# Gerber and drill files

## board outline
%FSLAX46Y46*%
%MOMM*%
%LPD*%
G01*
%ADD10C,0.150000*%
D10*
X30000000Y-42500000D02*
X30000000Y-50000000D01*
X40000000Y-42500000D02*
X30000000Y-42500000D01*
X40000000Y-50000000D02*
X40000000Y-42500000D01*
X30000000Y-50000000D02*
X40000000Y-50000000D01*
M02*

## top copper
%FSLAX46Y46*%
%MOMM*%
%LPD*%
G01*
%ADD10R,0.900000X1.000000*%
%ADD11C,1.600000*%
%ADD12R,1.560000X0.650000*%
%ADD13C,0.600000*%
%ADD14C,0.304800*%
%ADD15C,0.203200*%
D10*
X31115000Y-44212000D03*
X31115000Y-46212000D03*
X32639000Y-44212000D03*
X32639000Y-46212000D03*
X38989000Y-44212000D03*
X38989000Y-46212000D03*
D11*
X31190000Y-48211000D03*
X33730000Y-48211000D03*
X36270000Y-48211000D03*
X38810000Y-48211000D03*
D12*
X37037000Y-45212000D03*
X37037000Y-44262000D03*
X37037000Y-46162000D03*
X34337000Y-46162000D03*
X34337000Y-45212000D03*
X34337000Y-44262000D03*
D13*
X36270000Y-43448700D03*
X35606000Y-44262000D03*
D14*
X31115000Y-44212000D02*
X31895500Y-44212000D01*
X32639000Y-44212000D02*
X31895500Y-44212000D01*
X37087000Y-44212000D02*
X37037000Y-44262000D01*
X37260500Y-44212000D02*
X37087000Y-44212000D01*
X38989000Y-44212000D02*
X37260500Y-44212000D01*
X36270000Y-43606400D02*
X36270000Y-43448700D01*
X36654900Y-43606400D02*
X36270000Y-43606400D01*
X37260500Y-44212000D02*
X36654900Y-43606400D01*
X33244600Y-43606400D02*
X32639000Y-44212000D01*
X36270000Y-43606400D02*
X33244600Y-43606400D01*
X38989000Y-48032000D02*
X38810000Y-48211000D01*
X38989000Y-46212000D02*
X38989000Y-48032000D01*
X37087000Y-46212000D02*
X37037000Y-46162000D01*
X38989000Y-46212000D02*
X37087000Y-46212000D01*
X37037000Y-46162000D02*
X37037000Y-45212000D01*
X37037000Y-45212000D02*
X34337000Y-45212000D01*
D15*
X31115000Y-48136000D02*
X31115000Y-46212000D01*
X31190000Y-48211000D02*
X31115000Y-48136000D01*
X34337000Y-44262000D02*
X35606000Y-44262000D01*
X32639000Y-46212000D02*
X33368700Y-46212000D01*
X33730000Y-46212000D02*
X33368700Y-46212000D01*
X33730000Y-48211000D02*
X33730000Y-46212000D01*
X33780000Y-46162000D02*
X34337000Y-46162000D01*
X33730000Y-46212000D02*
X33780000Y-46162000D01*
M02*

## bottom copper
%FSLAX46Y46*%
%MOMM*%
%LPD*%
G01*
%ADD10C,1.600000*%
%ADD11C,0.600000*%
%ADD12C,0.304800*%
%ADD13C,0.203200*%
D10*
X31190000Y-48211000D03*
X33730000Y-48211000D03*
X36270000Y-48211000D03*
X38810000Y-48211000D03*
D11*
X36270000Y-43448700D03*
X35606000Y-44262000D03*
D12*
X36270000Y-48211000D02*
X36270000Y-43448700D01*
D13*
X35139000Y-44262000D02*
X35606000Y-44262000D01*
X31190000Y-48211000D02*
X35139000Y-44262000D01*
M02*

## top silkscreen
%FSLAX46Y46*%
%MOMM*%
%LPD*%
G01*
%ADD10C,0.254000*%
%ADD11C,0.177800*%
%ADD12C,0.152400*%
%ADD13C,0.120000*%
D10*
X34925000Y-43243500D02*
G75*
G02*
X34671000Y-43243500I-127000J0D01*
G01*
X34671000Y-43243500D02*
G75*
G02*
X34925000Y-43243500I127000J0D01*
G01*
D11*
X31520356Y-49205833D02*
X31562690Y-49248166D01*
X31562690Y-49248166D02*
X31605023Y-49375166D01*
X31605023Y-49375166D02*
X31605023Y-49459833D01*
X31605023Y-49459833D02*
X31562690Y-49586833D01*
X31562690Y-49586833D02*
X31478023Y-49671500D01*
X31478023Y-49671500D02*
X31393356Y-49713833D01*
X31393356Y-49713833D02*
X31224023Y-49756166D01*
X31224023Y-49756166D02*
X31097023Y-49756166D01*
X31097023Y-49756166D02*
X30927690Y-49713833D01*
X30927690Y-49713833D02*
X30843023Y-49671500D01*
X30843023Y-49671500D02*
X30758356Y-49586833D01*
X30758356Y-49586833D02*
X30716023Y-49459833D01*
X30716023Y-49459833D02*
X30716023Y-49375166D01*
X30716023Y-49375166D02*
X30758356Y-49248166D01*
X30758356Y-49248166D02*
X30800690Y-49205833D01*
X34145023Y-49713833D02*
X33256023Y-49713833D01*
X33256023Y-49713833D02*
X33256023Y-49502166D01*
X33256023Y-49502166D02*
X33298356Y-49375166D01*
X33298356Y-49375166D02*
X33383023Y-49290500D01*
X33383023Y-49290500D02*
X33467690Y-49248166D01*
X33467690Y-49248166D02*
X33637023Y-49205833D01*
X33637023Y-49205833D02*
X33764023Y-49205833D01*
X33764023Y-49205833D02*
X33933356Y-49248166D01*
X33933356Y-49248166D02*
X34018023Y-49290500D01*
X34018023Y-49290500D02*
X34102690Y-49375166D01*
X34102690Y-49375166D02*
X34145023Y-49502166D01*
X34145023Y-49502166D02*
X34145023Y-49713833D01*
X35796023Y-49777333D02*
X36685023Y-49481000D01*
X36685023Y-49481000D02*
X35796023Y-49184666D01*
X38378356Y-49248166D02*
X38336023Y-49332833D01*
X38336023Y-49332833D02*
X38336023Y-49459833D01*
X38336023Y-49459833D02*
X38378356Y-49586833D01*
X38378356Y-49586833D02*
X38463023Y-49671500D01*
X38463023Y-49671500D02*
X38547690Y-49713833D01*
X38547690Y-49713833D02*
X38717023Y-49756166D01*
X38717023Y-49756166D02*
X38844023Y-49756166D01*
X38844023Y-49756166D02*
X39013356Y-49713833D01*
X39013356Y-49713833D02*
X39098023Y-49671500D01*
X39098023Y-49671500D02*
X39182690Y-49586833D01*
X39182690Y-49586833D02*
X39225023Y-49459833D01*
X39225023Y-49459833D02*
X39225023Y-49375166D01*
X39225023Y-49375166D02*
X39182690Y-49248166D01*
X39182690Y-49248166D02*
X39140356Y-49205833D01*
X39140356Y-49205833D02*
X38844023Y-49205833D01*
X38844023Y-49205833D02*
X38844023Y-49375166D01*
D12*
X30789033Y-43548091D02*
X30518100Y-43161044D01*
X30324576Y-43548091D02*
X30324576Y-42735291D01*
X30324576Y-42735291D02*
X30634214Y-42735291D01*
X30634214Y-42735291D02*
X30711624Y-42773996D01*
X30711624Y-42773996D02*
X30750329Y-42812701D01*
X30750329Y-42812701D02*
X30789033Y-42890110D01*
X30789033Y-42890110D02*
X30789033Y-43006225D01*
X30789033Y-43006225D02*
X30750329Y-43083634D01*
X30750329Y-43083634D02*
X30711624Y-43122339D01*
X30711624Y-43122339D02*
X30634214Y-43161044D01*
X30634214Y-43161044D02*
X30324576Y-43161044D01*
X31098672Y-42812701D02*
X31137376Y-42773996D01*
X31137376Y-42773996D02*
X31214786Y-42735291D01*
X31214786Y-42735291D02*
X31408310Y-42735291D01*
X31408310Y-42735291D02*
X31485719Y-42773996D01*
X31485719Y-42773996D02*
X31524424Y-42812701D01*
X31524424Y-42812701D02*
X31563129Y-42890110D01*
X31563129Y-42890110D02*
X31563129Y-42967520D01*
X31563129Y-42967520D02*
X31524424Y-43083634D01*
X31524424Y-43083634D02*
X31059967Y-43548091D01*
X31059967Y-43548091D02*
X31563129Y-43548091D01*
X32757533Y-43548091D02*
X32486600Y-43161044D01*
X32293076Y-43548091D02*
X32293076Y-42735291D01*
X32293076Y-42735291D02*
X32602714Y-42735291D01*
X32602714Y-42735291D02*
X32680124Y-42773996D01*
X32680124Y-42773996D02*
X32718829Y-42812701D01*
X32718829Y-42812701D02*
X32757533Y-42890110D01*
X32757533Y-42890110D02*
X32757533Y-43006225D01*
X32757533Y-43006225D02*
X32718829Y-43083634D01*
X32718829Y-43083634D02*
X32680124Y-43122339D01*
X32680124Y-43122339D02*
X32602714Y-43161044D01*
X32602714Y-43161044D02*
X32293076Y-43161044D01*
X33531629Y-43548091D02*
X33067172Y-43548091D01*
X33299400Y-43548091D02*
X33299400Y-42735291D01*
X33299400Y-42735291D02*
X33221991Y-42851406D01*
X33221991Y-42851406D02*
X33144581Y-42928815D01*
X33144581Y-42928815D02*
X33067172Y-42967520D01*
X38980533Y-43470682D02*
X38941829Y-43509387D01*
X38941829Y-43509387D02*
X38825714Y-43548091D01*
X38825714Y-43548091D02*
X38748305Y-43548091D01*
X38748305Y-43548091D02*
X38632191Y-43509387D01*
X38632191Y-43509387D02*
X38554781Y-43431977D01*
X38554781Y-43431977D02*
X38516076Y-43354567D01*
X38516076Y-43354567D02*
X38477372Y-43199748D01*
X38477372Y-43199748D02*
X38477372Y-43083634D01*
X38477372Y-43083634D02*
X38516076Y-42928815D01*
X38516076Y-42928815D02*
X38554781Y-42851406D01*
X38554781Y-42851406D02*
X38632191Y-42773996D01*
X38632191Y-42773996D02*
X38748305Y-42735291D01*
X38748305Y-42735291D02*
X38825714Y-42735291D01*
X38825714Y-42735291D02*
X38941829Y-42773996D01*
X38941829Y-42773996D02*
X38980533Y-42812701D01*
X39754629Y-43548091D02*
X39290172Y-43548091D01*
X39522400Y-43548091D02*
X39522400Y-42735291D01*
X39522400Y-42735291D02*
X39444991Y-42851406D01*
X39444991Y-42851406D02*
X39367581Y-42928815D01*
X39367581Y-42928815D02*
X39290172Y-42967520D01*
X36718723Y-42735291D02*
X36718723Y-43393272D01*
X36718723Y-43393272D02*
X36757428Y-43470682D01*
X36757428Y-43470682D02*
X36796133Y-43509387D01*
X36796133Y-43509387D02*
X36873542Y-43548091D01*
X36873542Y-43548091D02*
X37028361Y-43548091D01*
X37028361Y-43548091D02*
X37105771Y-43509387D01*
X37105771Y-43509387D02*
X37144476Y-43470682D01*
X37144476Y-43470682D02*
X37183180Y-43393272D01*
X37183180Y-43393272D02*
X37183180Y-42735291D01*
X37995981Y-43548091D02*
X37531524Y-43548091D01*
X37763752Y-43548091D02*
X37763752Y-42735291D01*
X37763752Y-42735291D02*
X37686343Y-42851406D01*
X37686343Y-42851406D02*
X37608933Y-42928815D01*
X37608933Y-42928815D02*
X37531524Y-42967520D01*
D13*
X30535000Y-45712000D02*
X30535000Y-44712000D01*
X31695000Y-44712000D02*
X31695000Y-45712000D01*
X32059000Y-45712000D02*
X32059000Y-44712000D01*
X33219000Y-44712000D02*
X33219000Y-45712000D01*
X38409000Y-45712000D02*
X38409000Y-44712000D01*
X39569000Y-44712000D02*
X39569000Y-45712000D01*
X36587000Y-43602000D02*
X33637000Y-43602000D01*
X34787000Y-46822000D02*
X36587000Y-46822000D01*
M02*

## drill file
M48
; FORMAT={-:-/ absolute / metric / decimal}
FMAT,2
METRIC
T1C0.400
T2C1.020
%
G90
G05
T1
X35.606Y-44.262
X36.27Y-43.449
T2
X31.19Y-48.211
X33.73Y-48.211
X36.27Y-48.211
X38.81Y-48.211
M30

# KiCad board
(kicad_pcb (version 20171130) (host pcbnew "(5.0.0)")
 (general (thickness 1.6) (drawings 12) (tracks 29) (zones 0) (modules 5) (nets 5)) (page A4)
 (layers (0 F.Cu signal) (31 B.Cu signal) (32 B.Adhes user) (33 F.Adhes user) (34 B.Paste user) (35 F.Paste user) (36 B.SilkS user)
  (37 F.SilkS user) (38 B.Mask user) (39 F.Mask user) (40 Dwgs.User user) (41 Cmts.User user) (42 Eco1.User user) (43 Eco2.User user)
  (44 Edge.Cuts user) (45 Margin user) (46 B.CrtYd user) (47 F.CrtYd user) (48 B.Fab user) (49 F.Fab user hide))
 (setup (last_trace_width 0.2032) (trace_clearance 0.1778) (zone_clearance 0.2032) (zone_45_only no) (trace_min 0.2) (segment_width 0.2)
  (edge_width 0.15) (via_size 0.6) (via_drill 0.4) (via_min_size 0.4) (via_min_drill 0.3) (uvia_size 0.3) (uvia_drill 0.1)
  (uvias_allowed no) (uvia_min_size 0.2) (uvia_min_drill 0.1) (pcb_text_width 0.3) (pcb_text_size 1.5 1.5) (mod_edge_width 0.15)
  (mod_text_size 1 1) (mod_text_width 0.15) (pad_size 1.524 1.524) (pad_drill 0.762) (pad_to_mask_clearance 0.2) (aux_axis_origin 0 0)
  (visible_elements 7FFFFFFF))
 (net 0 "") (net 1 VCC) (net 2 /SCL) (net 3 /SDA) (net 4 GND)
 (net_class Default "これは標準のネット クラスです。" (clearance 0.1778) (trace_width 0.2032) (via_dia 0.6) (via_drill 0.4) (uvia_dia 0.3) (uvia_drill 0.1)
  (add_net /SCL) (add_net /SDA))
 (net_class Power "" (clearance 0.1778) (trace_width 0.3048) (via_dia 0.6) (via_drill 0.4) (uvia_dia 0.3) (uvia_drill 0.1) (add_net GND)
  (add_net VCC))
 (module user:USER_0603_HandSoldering (layer F.Cu) (at 31.115 45.212 270)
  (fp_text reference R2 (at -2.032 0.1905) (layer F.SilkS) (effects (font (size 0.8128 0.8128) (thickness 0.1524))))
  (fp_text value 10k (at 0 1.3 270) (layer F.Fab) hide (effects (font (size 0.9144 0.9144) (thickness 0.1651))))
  (fp_line (start 0.5 0.58) (end -0.5 0.58) (layer F.SilkS) (width 0.12))
  (fp_line (start -0.5 -0.58) (end 0.5 -0.58) (layer F.SilkS) (width 0.12))
  (pad 1 smd rect (at -1 0 270) (size 1 0.9) (layers F.Cu F.Paste F.Mask) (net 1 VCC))
  (pad 2 smd rect (at 1 0 270) (size 1 0.9) (layers F.Cu F.Paste F.Mask) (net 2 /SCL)))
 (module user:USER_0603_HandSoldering (layer F.Cu) (at 32.639 45.212 270)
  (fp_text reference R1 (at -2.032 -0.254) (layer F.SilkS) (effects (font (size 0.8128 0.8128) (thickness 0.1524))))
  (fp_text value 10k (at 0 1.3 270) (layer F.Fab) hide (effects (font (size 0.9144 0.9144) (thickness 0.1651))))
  (fp_line (start 0.5 0.58) (end -0.5 0.58) (layer F.SilkS) (width 0.12))
  (fp_line (start -0.5 -0.58) (end 0.5 -0.58) (layer F.SilkS) (width 0.12))
  (pad 1 smd rect (at -1 0 270) (size 1 0.9) (layers F.Cu F.Paste F.Mask) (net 1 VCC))
  (pad 2 smd rect (at 1 0 270) (size 1 0.9) (layers F.Cu F.Paste F.Mask) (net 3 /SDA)))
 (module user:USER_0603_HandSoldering (layer F.Cu) (at 38.989 45.212 270)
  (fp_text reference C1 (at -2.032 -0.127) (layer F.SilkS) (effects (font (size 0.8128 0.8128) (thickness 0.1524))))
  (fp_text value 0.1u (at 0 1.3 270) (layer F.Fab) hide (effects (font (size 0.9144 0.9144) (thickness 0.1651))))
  (fp_line (start 0.5 0.58) (end -0.5 0.58) (layer F.SilkS) (width 0.12))
  (fp_line (start -0.5 -0.58) (end 0.5 -0.58) (layer F.SilkS) (width 0.12))
  (pad 1 smd rect (at -1 0 270) (size 1 0.9) (layers F.Cu F.Paste F.Mask) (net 1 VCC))
  (pad 2 smd rect (at 1 0 270) (size 1 0.9) (layers F.Cu F.Paste F.Mask) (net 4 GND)))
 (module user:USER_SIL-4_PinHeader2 (layer B.Cu) (at 35 48.211)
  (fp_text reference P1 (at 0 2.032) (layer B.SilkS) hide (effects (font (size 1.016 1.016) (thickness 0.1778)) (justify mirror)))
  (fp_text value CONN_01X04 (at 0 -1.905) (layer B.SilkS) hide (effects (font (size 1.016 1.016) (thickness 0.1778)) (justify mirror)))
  (pad 1 thru_hole circle (at -3.81 0) (size 1.6 1.6) (drill 1.02) (layers *.Cu *.Mask B.SilkS) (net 2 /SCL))
  (pad 2 thru_hole circle (at -1.27 0) (size 1.6 1.6) (drill 1.02) (layers *.Cu *.Mask B.SilkS) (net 3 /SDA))
  (pad 3 thru_hole circle (at 1.27 0) (size 1.6 1.6) (drill 1.02) (layers *.Cu *.Mask B.SilkS) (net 1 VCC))
  (pad 4 thru_hole circle (at 3.81 0) (size 1.6 1.6) (drill 1.02) (layers *.Cu *.Mask B.SilkS) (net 4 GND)))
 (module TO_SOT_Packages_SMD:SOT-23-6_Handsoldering (layer F.Cu) (at 35.687 45.212)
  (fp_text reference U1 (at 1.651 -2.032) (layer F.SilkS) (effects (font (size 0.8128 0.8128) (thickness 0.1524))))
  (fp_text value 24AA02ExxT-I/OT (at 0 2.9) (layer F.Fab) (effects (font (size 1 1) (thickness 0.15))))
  (fp_line (start 0.9 -1.61) (end -2.05 -1.61) (layer F.SilkS) (width 0.12))
  (fp_line (start -0.9 1.61) (end 0.9 1.61) (layer F.SilkS) (width 0.12))
  (pad 5 smd rect (at 1.35 0) (size 1.56 0.65) (layers F.Cu F.Paste F.Mask) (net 4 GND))
  (pad 6 smd rect (at 1.35 -0.95) (size 1.56 0.65) (layers F.Cu F.Paste F.Mask) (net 1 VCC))
  (pad 4 smd rect (at 1.35 0.95) (size 1.56 0.65) (layers F.Cu F.Paste F.Mask) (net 4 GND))
  (pad 3 smd rect (at -1.35 0.95) (size 1.56 0.65) (layers F.Cu F.Paste F.Mask) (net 3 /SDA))
  (pad 2 smd rect (at -1.35 0) (size 1.56 0.65) (layers F.Cu F.Paste F.Mask) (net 4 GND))
  (pad 1 smd rect (at -1.35 -0.95) (size 1.56 0.65) (layers F.Cu F.Paste F.Mask) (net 2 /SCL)))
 (gr_circle (center 34.798 43.2435) (end 34.925 43.2435) (layer F.SilkS) (width 0.254))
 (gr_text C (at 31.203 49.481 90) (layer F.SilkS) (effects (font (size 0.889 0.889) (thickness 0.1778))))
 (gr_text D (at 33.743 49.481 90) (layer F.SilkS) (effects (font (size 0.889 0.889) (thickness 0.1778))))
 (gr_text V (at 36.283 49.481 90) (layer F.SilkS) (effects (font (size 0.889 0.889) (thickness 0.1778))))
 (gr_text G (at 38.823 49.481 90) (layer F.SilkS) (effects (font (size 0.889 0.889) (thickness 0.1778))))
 (gr_line (start 30 42.5) (end 30 50) (angle 90) (layer Edge.Cuts) (width 0.15))
 (gr_line (start 40 42.5) (end 30 42.5) (angle 90) (layer Edge.Cuts) (width 0.15))
 (gr_line (start 40 50) (end 40 42.5) (angle 90) (layer Edge.Cuts) (width 0.15))
 (gr_line (start 30 50) (end 40 50) (angle 90) (layer Edge.Cuts) (width 0.15))
 (via (at 36.27 43.4487) (size 0.6) (layers F.Cu B.Cu) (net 1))
 (segment (start 31.115 44.212) (end 31.8955 44.212) (width 0.3048) (layer F.Cu) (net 1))
 (segment (start 32.639 44.212) (end 31.8955 44.212) (width 0.3048) (layer F.Cu) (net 1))
 (segment (start 37.087 44.212) (end 37.037 44.262) (width 0.3048) (layer F.Cu) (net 1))
 (segment (start 37.2605 44.212) (end 37.087 44.212) (width 0.3048) (layer F.Cu) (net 1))
 (segment (start 38.989 44.212) (end 37.2605 44.212) (width 0.3048) (layer F.Cu) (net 1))
 (segment (start 36.27 48.211) (end 36.27 43.4487) (width 0.3048) (layer B.Cu) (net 1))
 (segment (start 36.27 43.6064) (end 36.27 43.4487) (width 0.3048) (layer F.Cu) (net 1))
 (segment (start 36.6549 43.6064) (end 36.27 43.6064) (width 0.3048) (layer F.Cu) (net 1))
 (segment (start 37.2605 44.212) (end 36.6549 43.6064) (width 0.3048) (layer F.Cu) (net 1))
 (segment (start 33.2446 43.6064) (end 32.639 44.212) (width 0.3048) (layer F.Cu) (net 1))
 (segment (start 36.27 43.6064) (end 33.2446 43.6064) (width 0.3048) (layer F.Cu) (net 1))
 (segment (start 38.989 48.032) (end 38.81 48.211) (width 0.3048) (layer F.Cu) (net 4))
 (segment (start 38.989 46.212) (end 38.989 48.032) (width 0.3048) (layer F.Cu) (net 4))
 (segment (start 37.087 46.212) (end 37.037 46.162) (width 0.3048) (layer F.Cu) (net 4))
 (segment (start 38.989 46.212) (end 37.087 46.212) (width 0.3048) (layer F.Cu) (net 4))
 (segment (start 37.037 46.162) (end 37.037 45.212) (width 0.3048) (layer F.Cu) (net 4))
 (segment (start 37.037 45.212) (end 34.337 45.212) (width 0.3048) (layer F.Cu) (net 4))
 (via (at 35.606 44.262) (size 0.6) (layers F.Cu B.Cu) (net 2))
 (segment (start 31.115 48.136) (end 31.115 46.212) (width 0.2032) (layer F.Cu) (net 2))
 (segment (start 31.19 48.211) (end 31.115 48.136) (width 0.2032) (layer F.Cu) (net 2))
 (segment (start 35.139 44.262) (end 35.606 44.262) (width 0.2032) (layer B.Cu) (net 2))
 (segment (start 31.19 48.211) (end 35.139 44.262) (width 0.2032) (layer B.Cu) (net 2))
 (segment (start 34.337 44.262) (end 35.606 44.262) (width 0.2032) (layer F.Cu) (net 2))
 (segment (start 32.639 46.212) (end 33.3687 46.212) (width 0.2032) (layer F.Cu) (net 3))
 (segment (start 33.73 46.212) (end 33.3687 46.212) (width 0.2032) (layer F.Cu) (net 3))
 (segment (start 33.73 48.211) (end 33.73 46.212) (width 0.2032) (layer F.Cu) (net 3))
 (segment (start 33.78 46.162) (end 34.337 46.162) (width 0.2032) (layer F.Cu) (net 3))
 (segment (start 33.73 46.212) (end 33.78 46.162) (width 0.2032) (layer F.Cu) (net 3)))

